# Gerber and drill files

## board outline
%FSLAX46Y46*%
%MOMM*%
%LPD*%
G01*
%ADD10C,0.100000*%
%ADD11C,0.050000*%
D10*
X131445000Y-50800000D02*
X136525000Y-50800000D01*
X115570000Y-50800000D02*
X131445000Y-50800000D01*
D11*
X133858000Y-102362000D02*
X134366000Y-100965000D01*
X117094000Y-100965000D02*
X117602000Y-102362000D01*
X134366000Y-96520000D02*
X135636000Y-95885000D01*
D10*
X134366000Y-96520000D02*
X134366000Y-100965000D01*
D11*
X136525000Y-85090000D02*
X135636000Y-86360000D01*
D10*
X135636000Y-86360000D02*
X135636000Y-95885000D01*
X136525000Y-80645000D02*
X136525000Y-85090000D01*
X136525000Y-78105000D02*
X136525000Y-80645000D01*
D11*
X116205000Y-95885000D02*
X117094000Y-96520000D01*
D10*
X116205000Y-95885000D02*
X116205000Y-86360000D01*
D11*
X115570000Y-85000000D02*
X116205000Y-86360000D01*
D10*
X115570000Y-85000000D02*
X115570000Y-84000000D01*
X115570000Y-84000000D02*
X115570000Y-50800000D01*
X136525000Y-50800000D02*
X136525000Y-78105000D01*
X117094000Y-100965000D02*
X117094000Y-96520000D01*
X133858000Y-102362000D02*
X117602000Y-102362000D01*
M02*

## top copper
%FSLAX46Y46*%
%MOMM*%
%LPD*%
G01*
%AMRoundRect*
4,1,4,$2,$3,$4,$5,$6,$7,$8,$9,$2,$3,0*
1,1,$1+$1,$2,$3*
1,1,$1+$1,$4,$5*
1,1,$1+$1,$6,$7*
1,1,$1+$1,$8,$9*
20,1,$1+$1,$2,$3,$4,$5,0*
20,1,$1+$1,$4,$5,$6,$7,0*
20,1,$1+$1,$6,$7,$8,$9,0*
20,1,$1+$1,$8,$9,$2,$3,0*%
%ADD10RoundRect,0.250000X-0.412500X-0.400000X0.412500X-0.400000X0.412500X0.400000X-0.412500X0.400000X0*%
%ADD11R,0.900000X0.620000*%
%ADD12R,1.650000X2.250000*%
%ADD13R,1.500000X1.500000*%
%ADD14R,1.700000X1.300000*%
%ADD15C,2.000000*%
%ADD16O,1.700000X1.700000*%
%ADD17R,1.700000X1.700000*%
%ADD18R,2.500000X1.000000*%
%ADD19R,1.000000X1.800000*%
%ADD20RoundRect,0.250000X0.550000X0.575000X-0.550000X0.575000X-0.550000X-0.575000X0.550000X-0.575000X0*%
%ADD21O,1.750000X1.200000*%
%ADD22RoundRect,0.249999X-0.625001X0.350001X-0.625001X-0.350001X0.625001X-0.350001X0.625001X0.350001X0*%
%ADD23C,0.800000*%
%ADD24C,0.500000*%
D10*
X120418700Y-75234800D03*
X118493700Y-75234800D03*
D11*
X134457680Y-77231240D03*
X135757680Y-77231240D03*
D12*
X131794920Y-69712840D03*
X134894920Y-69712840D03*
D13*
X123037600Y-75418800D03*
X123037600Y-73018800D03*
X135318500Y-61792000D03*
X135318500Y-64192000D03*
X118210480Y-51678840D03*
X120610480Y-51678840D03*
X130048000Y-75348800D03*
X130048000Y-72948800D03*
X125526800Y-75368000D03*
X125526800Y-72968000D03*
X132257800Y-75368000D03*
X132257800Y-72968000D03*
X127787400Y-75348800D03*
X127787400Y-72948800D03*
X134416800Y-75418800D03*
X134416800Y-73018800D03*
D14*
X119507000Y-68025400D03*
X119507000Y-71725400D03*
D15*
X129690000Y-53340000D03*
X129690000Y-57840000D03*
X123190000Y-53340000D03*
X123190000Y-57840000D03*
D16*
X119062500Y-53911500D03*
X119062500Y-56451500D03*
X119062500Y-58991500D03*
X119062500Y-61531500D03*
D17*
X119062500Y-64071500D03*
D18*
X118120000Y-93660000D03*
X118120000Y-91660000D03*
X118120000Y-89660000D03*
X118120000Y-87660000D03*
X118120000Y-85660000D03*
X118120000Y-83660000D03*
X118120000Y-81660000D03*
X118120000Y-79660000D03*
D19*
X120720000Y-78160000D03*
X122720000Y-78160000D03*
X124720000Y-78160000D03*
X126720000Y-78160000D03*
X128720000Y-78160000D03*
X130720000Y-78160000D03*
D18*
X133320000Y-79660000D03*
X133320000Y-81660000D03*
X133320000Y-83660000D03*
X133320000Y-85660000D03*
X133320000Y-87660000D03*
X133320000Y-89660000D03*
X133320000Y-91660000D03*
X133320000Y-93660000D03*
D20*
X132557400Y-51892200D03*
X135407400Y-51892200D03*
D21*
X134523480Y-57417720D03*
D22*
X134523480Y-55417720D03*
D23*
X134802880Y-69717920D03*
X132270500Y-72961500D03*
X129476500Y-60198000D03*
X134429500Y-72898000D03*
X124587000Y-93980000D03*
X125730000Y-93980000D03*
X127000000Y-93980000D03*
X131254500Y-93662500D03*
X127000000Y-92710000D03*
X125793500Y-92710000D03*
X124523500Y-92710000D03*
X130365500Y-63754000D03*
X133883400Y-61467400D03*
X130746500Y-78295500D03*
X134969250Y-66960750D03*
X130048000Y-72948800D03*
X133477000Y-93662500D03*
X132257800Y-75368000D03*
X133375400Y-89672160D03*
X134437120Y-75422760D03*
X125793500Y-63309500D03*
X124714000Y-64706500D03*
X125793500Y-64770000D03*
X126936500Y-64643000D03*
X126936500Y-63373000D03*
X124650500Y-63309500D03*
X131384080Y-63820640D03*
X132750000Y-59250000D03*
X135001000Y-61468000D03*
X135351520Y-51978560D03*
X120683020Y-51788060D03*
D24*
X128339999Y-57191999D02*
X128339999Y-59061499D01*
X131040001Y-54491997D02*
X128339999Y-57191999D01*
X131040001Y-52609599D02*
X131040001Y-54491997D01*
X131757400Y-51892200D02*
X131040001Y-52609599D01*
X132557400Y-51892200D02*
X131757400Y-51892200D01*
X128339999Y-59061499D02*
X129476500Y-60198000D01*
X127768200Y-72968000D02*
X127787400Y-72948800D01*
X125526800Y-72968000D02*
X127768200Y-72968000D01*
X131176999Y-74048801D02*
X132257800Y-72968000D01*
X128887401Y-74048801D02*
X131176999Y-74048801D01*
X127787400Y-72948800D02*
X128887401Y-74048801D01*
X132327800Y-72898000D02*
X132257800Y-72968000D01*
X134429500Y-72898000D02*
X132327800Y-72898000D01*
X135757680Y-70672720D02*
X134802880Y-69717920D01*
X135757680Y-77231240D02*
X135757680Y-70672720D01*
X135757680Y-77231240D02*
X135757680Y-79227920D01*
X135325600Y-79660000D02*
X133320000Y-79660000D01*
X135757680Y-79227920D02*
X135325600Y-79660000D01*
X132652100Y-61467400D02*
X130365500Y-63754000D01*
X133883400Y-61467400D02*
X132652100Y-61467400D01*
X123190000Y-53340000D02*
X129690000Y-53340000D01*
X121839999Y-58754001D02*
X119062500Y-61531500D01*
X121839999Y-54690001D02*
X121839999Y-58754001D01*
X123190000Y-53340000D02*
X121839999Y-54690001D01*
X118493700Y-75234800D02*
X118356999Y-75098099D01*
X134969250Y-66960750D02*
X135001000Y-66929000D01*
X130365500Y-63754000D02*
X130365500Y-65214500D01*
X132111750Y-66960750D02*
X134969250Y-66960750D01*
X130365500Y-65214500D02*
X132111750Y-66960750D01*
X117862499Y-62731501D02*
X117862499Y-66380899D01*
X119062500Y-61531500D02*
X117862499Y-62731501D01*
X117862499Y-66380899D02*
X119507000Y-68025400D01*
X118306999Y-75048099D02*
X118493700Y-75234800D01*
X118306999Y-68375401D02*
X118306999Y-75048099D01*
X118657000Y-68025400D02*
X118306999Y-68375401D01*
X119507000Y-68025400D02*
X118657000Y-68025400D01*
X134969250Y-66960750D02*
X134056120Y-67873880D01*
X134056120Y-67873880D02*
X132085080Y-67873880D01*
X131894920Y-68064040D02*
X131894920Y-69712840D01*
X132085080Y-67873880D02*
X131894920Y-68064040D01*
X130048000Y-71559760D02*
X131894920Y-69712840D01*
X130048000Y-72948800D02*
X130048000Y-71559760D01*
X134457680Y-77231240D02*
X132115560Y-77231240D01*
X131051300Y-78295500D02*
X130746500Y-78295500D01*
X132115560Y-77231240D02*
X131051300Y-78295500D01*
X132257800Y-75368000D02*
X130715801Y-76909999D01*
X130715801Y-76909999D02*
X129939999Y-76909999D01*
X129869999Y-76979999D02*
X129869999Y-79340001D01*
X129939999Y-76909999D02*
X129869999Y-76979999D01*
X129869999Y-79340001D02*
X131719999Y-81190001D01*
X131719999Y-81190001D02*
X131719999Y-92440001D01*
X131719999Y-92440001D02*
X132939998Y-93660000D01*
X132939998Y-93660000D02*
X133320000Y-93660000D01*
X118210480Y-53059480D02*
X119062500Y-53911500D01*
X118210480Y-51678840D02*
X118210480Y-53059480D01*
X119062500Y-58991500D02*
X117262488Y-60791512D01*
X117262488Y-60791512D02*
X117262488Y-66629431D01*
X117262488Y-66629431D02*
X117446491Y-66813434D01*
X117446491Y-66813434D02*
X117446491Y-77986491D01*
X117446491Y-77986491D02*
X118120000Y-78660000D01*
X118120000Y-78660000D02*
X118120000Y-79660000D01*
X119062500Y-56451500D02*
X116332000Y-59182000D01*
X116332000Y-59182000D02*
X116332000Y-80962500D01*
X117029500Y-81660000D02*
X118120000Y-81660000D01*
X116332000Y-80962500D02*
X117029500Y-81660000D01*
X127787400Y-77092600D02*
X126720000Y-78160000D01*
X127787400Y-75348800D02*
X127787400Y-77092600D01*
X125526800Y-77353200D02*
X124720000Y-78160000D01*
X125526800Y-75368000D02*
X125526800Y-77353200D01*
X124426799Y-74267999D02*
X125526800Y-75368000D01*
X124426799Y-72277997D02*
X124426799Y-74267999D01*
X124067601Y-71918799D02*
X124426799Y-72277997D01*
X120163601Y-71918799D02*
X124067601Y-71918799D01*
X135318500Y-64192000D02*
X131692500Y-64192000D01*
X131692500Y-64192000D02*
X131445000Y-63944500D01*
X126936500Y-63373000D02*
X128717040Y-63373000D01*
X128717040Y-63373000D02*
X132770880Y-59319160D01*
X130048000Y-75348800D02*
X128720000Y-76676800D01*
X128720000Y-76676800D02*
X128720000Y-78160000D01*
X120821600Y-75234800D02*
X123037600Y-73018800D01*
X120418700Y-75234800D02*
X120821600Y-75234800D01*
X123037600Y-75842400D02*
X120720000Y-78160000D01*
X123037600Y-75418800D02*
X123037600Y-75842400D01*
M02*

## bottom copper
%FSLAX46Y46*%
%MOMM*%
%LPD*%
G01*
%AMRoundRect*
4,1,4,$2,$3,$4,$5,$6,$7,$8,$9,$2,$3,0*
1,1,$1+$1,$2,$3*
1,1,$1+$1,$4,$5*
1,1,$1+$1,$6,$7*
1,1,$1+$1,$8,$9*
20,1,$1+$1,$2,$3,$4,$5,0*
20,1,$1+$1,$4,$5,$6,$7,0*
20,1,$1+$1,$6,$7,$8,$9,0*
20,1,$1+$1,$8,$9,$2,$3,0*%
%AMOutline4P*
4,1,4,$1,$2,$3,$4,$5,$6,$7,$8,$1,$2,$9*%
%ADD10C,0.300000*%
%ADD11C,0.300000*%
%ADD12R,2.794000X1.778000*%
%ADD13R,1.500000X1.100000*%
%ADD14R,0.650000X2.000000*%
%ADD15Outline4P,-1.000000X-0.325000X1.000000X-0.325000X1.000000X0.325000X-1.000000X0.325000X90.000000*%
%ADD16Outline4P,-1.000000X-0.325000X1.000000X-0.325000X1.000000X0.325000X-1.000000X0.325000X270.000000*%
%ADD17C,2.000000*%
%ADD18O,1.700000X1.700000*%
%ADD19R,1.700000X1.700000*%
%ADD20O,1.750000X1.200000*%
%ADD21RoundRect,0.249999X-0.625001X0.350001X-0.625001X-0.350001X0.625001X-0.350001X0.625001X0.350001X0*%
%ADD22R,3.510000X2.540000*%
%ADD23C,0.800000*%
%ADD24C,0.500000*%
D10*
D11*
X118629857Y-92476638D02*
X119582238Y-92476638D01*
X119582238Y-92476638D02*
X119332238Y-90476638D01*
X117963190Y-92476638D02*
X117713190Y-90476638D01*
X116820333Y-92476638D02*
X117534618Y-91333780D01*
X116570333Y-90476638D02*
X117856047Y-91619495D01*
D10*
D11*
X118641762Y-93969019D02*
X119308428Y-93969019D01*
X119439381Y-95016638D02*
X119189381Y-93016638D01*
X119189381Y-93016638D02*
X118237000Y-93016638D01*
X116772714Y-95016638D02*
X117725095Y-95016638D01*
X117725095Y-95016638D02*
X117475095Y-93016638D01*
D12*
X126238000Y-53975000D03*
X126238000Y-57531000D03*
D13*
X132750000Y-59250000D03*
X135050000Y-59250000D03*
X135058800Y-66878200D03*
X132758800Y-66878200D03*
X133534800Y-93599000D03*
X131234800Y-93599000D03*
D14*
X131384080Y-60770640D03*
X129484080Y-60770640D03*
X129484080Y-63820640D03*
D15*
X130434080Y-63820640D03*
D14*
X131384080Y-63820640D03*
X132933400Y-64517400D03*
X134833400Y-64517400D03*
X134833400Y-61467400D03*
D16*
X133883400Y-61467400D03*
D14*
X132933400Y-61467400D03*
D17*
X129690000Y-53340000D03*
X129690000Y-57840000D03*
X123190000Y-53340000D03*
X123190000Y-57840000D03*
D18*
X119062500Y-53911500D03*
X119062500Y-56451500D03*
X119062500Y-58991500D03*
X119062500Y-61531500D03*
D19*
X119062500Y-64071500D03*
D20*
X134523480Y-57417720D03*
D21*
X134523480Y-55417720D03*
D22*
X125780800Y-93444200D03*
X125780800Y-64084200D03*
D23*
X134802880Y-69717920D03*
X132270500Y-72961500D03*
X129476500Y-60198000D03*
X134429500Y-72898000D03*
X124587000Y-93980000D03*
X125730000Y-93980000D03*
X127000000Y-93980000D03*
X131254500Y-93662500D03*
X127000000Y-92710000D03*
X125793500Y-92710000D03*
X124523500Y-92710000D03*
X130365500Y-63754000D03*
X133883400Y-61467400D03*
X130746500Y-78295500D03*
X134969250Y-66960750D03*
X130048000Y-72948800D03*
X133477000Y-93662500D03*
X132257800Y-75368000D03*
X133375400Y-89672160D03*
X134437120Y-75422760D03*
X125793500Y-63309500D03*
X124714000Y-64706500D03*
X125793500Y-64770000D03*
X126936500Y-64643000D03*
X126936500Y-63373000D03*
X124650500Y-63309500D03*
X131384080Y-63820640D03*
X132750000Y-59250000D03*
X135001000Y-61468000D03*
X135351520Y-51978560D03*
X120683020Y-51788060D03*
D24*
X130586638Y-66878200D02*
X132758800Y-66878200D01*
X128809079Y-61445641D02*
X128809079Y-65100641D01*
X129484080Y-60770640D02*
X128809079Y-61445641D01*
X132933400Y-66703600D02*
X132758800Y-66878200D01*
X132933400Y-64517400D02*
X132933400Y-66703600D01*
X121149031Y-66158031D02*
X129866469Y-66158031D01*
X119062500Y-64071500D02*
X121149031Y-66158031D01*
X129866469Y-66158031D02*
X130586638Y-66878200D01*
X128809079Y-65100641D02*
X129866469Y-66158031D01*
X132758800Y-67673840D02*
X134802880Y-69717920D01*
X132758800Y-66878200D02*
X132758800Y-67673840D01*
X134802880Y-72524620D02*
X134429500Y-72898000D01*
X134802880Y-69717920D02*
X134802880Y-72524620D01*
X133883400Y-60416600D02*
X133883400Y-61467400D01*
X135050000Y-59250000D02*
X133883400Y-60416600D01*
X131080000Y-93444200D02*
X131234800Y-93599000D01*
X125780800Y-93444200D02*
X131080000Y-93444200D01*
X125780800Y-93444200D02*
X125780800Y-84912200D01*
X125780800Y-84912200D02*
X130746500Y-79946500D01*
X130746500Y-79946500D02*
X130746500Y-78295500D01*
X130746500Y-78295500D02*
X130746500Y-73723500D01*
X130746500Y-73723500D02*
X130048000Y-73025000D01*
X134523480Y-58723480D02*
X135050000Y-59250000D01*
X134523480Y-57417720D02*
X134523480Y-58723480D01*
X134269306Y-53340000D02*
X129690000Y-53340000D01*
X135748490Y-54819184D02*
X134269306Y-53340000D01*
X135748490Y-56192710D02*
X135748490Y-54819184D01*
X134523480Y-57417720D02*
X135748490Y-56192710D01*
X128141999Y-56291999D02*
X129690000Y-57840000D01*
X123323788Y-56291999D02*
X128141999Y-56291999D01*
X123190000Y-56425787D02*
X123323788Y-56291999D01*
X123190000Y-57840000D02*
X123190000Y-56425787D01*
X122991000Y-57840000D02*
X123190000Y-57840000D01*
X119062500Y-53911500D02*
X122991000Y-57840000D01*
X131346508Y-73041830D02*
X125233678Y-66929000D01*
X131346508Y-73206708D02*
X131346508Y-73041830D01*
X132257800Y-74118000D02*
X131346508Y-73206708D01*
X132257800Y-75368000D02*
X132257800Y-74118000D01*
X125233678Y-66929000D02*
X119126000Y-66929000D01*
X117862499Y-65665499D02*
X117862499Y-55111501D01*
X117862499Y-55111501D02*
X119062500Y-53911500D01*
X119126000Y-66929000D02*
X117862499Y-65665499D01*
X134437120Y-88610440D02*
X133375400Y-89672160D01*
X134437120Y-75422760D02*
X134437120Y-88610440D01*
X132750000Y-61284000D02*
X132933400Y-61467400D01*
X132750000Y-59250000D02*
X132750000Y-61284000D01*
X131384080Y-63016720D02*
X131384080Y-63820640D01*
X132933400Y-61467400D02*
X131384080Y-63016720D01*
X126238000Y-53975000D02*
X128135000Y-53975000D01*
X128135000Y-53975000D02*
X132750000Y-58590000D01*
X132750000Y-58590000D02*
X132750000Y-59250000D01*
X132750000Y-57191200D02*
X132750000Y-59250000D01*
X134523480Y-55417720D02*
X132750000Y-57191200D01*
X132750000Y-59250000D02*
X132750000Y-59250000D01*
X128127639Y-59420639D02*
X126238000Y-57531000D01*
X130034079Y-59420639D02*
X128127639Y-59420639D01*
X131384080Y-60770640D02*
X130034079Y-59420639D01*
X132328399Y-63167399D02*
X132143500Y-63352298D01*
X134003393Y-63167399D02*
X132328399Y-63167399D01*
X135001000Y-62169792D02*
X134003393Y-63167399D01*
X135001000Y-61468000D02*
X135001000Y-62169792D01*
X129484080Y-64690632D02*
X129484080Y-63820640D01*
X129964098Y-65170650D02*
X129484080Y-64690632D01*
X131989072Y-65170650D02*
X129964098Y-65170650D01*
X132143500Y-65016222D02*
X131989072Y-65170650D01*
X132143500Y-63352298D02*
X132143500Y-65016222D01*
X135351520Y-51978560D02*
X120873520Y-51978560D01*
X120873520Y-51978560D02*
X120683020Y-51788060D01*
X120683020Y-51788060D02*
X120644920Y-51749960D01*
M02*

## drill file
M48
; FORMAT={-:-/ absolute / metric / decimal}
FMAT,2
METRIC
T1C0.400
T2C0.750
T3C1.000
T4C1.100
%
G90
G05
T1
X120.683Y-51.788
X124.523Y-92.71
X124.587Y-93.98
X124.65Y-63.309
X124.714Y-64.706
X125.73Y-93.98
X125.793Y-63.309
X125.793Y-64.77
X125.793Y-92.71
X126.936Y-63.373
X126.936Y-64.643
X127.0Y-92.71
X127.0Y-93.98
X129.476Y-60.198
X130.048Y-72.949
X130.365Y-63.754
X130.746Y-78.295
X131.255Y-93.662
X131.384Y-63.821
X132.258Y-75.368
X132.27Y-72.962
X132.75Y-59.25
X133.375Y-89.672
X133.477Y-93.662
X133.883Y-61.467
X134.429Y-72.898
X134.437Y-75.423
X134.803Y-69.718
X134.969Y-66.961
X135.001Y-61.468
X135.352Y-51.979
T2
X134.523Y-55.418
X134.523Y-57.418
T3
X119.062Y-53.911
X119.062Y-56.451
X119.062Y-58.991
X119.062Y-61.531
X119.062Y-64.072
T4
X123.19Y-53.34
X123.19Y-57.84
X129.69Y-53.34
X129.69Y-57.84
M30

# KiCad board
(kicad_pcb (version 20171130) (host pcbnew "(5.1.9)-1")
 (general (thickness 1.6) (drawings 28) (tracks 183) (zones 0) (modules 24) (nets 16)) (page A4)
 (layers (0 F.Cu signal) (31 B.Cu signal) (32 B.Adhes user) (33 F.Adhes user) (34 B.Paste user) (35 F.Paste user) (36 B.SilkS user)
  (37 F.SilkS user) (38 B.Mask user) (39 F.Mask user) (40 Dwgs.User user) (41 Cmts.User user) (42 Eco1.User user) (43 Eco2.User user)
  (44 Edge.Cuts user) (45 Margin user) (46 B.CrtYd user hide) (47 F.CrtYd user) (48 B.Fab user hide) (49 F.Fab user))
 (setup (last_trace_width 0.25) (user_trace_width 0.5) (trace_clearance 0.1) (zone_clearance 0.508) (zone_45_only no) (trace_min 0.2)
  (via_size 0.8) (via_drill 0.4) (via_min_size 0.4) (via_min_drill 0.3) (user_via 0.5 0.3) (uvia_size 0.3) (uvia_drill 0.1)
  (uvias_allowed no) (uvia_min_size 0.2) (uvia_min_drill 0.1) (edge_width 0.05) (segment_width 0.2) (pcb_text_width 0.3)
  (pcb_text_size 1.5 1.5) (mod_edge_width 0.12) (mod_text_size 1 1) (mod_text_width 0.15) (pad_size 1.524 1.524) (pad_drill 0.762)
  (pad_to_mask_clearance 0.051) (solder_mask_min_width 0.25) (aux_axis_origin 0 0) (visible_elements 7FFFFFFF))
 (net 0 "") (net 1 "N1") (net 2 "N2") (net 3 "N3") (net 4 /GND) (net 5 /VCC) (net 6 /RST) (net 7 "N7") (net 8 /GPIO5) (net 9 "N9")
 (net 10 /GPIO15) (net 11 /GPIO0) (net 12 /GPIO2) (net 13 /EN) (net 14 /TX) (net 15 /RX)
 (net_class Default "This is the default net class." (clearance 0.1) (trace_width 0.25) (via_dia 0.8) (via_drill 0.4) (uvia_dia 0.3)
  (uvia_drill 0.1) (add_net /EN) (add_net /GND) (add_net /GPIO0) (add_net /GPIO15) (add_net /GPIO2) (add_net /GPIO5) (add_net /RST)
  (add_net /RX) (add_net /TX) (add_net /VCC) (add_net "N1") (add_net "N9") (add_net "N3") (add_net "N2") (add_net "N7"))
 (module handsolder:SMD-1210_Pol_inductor (layer B.Cu) (at 126.238 55.753 270)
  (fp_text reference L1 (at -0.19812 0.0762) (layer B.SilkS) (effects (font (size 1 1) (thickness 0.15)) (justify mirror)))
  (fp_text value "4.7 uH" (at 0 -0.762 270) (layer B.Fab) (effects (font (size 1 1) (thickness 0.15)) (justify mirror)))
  (pad 1 smd rect (at -1.778 0 270) (size 1.778 2.794) (layers B.Cu B.Paste B.Mask) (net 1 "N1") (zone_connect 2))
  (pad 2 smd rect (at 1.778 0 270) (size 1.778 2.794) (layers B.Cu B.Paste B.Mask) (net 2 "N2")))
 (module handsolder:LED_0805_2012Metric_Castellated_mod (layer F.Cu) (at 119.4562 75.2348)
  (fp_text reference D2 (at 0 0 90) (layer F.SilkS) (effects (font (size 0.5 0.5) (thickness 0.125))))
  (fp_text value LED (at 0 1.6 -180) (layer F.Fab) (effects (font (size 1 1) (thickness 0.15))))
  (pad 2 smd roundrect (at 0.9625 0) (size 1.325 1.3) (layers F.Cu F.Paste F.Mask) (roundrect_rratio 0.1923076923076923) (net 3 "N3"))
  (pad 1 smd roundrect (at -0.9625 0) (size 1.325 1.3) (layers F.Cu F.Paste F.Mask) (roundrect_rratio 0.1923076923076923) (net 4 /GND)))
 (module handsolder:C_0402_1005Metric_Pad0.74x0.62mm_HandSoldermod (layer F.Cu) (at 135.10768 77.23124 180)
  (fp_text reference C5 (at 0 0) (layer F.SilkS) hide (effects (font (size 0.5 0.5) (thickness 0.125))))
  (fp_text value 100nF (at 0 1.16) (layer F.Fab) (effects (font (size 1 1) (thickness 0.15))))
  (pad 2 smd rect (at 0.65 0 180) (size 0.9 0.62) (layers F.Cu F.Paste F.Mask) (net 4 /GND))
  (pad 1 smd rect (at -0.65 0 180) (size 0.9 0.62) (layers F.Cu F.Paste F.Mask) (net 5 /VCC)))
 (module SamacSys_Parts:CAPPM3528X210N (layer F.Cu) (at 133.34492 69.71284 180)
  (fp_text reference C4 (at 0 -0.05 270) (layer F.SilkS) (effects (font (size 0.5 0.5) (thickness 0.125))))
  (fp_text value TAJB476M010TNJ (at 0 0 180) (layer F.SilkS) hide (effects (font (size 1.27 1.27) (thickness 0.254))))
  (pad 2 smd rect (at 1.55 0 180) (size 1.65 2.25) (layers F.Cu F.Paste F.Mask) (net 4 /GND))
  (pad 1 smd rect (at -1.55 0 180) (size 1.65 2.25) (layers F.Cu F.Paste F.Mask) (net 5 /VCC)))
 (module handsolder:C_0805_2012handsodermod (layer B.Cu) (at 133.9 59.25 180)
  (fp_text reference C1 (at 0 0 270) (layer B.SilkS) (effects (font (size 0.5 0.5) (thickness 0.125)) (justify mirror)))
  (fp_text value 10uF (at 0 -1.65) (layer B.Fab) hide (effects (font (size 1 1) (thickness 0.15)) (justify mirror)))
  (pad 2 smd rect (at 1.15 0 180) (size 1.5 1.1) (layers B.Cu B.Paste B.Mask) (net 1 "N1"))
  (pad 1 smd rect (at -1.15 0 180) (size 1.5 1.1) (layers B.Cu B.Paste B.Mask) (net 4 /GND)))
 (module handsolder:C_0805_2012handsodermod (layer B.Cu) (at 133.9088 66.8782)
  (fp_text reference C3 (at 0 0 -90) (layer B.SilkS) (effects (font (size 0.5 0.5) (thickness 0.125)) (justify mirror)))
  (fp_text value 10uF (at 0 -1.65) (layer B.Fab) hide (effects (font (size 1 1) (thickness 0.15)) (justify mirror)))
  (pad 2 smd rect (at 1.15 0) (size 1.5 1.1) (layers B.Cu B.Paste B.Mask) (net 4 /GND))
  (pad 1 smd rect (at -1.15 0) (size 1.5 1.1) (layers B.Cu B.Paste B.Mask) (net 5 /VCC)))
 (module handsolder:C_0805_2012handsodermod (layer B.Cu) (at 132.3848 93.599)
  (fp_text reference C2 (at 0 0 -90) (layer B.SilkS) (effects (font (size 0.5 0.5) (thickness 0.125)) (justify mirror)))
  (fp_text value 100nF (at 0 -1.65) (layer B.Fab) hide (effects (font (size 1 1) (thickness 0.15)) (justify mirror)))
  (pad 2 smd rect (at 1.15 0) (size 1.5 1.1) (layers B.Cu B.Paste B.Mask) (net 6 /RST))
  (pad 1 smd rect (at -1.15 0) (size 1.5 1.1) (layers B.Cu B.Paste B.Mask) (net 4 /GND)))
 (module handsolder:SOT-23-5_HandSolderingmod (layer B.Cu) (at 130.43408 62.27064 90)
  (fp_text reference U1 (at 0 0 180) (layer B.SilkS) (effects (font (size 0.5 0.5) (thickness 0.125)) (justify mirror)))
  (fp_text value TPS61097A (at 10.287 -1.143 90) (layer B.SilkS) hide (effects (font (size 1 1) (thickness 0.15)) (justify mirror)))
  (pad 5 smd rect (at 1.5 0.95 90) (size 2 0.65) (layers B.Cu B.Paste B.Mask) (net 2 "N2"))
  (pad 4 smd rect (at 1.5 -0.95 90) (size 2 0.65) (layers B.Cu B.Paste B.Mask) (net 5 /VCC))
  (pad 3 smd rect (at -1.55 -0.95 90) (size 2 0.65) (layers B.Cu B.Paste B.Mask) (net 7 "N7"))
  (pad 2 smd trapezoid (at -1.55 0 90) (size 2 0.65) (layers B.Cu B.Paste B.Mask) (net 4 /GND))
  (pad 1 smd rect (at -1.55 0.95 90) (size 2 0.65) (layers B.Cu B.Paste B.Mask) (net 1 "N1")))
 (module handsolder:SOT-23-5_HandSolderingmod (layer B.Cu) (at 133.8834 63.0174 270)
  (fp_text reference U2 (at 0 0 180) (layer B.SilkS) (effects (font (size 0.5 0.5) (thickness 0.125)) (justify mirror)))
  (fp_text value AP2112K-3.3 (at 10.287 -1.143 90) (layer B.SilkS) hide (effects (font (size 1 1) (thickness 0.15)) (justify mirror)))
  (pad 5 smd rect (at 1.5 0.95 270) (size 2 0.65) (layers B.Cu B.Paste B.Mask) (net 5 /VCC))
  (pad 4 smd rect (at 1.5 -0.95 270) (size 2 0.65) (layers B.Cu B.Paste B.Mask))
  (pad 3 smd rect (at -1.55 -0.95 270) (size 2 0.65) (layers B.Cu B.Paste B.Mask) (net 7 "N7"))
  (pad 2 smd trapezoid (at -1.55 0 270) (size 2 0.65) (layers B.Cu B.Paste B.Mask) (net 4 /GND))
  (pad 1 smd rect (at -1.55 0.95 270) (size 2 0.65) (layers B.Cu B.Paste B.Mask) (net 1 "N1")))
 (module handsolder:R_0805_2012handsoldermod (layer F.Cu) (at 123.0376 74.2188 270)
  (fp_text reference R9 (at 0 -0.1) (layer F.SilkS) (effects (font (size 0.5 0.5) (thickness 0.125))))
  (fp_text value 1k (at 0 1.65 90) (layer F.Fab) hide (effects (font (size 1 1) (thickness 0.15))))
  (pad 2 smd rect (at 1.2 0 270) (size 1.5 1.5) (layers F.Cu F.Paste F.Mask) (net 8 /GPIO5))
  (pad 1 smd rect (at -1.2 0 270) (size 1.5 1.5) (layers F.Cu F.Paste F.Mask) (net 3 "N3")))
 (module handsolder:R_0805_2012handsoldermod (layer F.Cu) (at 135.3185 62.992 90)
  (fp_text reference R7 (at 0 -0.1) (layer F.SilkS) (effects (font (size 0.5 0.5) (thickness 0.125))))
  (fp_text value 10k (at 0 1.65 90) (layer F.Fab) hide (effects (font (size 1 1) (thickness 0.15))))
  (pad 2 smd rect (at 1.2 0 90) (size 1.5 1.5) (layers F.Cu F.Paste F.Mask) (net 7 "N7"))
  (pad 1 smd rect (at -1.2 0 90) (size 1.5 1.5) (layers F.Cu F.Paste F.Mask) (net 1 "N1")))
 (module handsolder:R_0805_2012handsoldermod (layer F.Cu) (at 119.41048 51.67884 180)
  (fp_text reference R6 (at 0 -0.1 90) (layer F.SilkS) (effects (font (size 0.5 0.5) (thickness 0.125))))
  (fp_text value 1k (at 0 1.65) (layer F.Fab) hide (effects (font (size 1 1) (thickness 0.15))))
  (pad 2 smd rect (at 1.2 0 180) (size 1.5 1.5) (layers F.Cu F.Paste F.Mask) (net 6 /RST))
  (pad 1 smd rect (at -1.2 0 180) (size 1.5 1.5) (layers F.Cu F.Paste F.Mask) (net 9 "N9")))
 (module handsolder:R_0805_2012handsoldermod (layer F.Cu) (at 130.048 74.1488 270)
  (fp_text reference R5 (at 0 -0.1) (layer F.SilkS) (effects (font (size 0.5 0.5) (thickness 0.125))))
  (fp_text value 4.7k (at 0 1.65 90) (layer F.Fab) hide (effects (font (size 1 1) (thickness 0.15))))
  (pad 2 smd rect (at 1.2 0 270) (size 1.5 1.5) (layers F.Cu F.Paste F.Mask) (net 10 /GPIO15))
  (pad 1 smd rect (at -1.2 0 270) (size 1.5 1.5) (layers F.Cu F.Paste F.Mask) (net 4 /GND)))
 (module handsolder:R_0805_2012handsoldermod (layer F.Cu) (at 125.5268 74.168 270)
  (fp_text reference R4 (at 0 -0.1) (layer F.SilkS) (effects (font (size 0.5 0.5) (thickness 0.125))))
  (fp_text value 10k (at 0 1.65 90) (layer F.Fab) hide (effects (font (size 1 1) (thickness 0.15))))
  (pad 2 smd rect (at 1.2 0 270) (size 1.5 1.5) (layers F.Cu F.Paste F.Mask) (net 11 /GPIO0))
  (pad 1 smd rect (at -1.2 0 270) (size 1.5 1.5) (layers F.Cu F.Paste F.Mask) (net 5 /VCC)))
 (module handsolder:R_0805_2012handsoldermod (layer F.Cu) (at 132.2578 74.168 270)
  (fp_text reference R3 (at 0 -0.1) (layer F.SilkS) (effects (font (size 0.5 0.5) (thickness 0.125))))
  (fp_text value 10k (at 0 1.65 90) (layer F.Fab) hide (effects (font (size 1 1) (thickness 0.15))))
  (pad 2 smd rect (at 1.2 0 270) (size 1.5 1.5) (layers F.Cu F.Paste F.Mask) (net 6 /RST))
  (pad 1 smd rect (at -1.2 0 270) (size 1.5 1.5) (layers F.Cu F.Paste F.Mask) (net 5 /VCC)))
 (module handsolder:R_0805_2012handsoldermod (layer F.Cu) (at 127.7874 74.1488 270)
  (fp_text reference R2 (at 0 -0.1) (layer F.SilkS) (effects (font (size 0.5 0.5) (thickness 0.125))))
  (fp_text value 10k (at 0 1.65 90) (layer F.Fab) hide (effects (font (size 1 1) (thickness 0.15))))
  (pad 2 smd rect (at 1.2 0 270) (size 1.5 1.5) (layers F.Cu F.Paste F.Mask) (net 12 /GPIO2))
  (pad 1 smd rect (at -1.2 0 270) (size 1.5 1.5) (layers F.Cu F.Paste F.Mask) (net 5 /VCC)))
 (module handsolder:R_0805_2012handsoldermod (layer F.Cu) (at 134.4168 74.2188 270)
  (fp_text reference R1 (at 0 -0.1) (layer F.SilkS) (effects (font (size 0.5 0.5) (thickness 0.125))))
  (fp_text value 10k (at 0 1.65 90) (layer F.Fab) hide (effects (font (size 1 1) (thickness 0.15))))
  (pad 2 smd rect (at 1.2 0 270) (size 1.5 1.5) (layers F.Cu F.Paste F.Mask) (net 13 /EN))
  (pad 1 smd rect (at -1.2 0 270) (size 1.5 1.5) (layers F.Cu F.Paste F.Mask) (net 5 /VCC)))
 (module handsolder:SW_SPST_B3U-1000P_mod (layer F.Cu) (at 119.507 69.8754 90)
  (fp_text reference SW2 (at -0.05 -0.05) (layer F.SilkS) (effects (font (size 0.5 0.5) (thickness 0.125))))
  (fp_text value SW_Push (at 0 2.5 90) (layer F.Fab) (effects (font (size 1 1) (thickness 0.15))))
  (pad 2 smd rect (at 1.85 0 90) (size 1.3 1.7) (layers F.Cu F.Paste F.Mask) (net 4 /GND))
  (pad 1 smd rect (at -1.85 0 90) (size 1.3 1.7) (layers F.Cu F.Paste F.Mask) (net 11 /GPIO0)))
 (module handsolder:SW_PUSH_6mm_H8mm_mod (layer F.Cu) (at 123.19 53.34)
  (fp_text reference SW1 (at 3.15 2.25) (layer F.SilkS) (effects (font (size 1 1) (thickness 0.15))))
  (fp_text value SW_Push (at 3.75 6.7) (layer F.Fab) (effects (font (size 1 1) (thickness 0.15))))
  (pad 1 thru_hole circle (at 6.5 0 90) (size 2 2) (drill 1.1) (layers *.Cu *.Mask) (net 4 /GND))
  (pad 2 thru_hole circle (at 6.5 4.5 90) (size 2 2) (drill 1.1) (layers *.Cu *.Mask) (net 6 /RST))
  (pad 1 thru_hole circle (at 0 0 90) (size 2 2) (drill 1.1) (layers *.Cu *.Mask) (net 4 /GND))
  (pad 2 thru_hole circle (at 0 4.5 90) (size 2 2) (drill 1.1) (layers *.Cu *.Mask) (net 6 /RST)))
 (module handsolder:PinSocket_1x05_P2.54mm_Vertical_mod (layer F.Cu) (at 119.0625 64.0715 180)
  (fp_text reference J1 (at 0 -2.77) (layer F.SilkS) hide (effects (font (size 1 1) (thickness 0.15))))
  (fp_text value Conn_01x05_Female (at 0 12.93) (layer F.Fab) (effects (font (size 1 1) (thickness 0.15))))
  (pad 5 thru_hole oval (at 0 10.16 180) (size 1.7 1.7) (drill 1) (layers *.Cu *.Mask) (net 6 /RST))
  (pad 4 thru_hole oval (at 0 7.62 180) (size 1.7 1.7) (drill 1) (layers *.Cu *.Mask) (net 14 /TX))
  (pad 3 thru_hole oval (at 0 5.08 180) (size 1.7 1.7) (drill 1) (layers *.Cu *.Mask) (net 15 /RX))
  (pad 2 thru_hole oval (at 0 2.54 180) (size 1.7 1.7) (drill 1) (layers *.Cu *.Mask) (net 4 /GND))
  (pad 1 thru_hole rect (at 0 0 180) (size 1.7 1.7) (drill 1) (layers *.Cu *.Mask) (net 5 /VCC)))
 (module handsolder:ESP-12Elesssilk (layer F.Cu) (at 125.72 90.16 180)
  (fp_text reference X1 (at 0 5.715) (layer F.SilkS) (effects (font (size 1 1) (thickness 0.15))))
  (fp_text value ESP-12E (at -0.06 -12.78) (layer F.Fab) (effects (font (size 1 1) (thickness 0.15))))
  (pad 22 smd rect (at 7.6 -3.5 180) (size 2.5 1) (layers F.Cu F.Paste F.Mask))
  (pad 21 smd rect (at 7.6 -1.5 180) (size 2.5 1) (layers F.Cu F.Paste F.Mask))
  (pad 20 smd rect (at 7.6 0.5 180) (size 2.5 1) (layers F.Cu F.Paste F.Mask))
  (pad 19 smd rect (at 7.6 2.5 180) (size 2.5 1) (layers F.Cu F.Paste F.Mask))
  (pad 18 smd rect (at 7.6 4.5 180) (size 2.5 1) (layers F.Cu F.Paste F.Mask))
  (pad 17 smd rect (at 7.6 6.5 180) (size 2.5 1) (layers F.Cu F.Paste F.Mask))
  (pad 16 smd rect (at 7.6 8.5 180) (size 2.5 1) (layers F.Cu F.Paste F.Mask) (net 14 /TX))
  (pad 15 smd rect (at 7.6 10.5 180) (size 2.5 1) (layers F.Cu F.Paste F.Mask) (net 15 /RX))
  (pad 14 smd rect (at 5 12 180) (size 1 1.8) (layers F.Cu F.Paste F.Mask) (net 8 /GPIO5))
  (pad 13 smd rect (at 3 12 180) (size 1 1.8) (layers F.Cu F.Paste F.Mask))
  (pad 12 smd rect (at 1 12 180) (size 1 1.8) (layers F.Cu F.Paste F.Mask) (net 11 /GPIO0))
  (pad 11 smd rect (at -1 12 180) (size 1 1.8) (layers F.Cu F.Paste F.Mask) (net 12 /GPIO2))
  (pad 10 smd rect (at -3 12 180) (size 1 1.8) (layers F.Cu F.Paste F.Mask) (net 10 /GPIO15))
  (pad 9 smd rect (at -5 12 180) (size 1 1.8) (layers F.Cu F.Paste F.Mask) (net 4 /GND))
  (pad 8 smd rect (at -7.6 10.5 180) (size 2.5 1) (layers F.Cu F.Paste F.Mask) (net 5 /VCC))
  (pad 7 smd rect (at -7.6 8.5 180) (size 2.5 1) (layers F.Cu F.Paste F.Mask))
  (pad 6 smd rect (at -7.6 6.5 180) (size 2.5 1) (layers F.Cu F.Paste F.Mask))
  (pad 5 smd rect (at -7.6 4.5 180) (size 2.5 1) (layers F.Cu F.Paste F.Mask))
  (pad 4 smd rect (at -7.6 2.5 180) (size 2.5 1) (layers F.Cu F.Paste F.Mask))
  (pad 3 smd rect (at -7.6 0.5 180) (size 2.5 1) (layers F.Cu F.Paste F.Mask) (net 13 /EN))
  (pad 2 smd rect (at -7.6 -1.5 180) (size 2.5 1) (layers F.Cu F.Paste F.Mask))
  (pad 1 smd rect (at -7.6 -3.5 180) (size 2.5 1) (layers F.Cu F.Paste F.Mask) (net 6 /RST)))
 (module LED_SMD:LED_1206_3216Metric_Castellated (layer F.Cu) (at 133.9824 51.8922 180)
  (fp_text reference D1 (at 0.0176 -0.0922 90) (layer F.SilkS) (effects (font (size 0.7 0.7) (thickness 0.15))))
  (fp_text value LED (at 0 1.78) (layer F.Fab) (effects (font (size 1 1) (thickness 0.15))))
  (pad 2 smd roundrect (at 1.425 0 180) (size 1.6 1.65) (layers F.Cu F.Paste F.Mask) (roundrect_rratio 0.15625) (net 5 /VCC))
  (pad 1 smd roundrect (at -1.425 0 180) (size 1.6 1.65) (layers F.Cu F.Paste F.Mask) (roundrect_rratio 0.15625) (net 9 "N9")))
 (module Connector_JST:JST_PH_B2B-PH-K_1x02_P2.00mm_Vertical (layer F.Cu) (at 134.52348 55.41772 270)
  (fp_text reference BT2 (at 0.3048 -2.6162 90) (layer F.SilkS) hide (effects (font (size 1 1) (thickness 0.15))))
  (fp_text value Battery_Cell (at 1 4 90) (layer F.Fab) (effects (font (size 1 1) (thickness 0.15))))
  (pad 2 thru_hole oval (at 2 0 270) (size 1.2 1.75) (drill 0.75) (layers *.Cu *.Mask) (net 4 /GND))
  (pad 1 thru_hole roundrect (at 0 0 270) (size 1.2 1.75) (drill 0.75) (layers *.Cu *.Mask) (roundrect_rratio 0.2083325) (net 1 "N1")))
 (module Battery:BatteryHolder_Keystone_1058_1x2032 (layer B.Cu) (at 125.7808 78.7642 270)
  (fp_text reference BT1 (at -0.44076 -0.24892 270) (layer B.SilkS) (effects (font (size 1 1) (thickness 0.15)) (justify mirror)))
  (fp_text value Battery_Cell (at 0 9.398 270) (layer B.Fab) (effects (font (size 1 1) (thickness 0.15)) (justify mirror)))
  (pad 2 smd rect (at 14.68 0 270) (size 2.54 3.51) (layers B.Cu B.Paste B.Mask) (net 4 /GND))
  (pad 1 smd rect (at -14.68 0 270) (size 2.54 3.51) (layers B.Cu B.Paste B.Mask) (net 1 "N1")))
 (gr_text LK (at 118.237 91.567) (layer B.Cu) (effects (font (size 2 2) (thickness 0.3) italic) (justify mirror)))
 (gr_line (start 131.445 50.8) (end 136.525 50.8) (layer Edge.Cuts) (width 0.1))
 (gr_line (start 115.57 50.8) (end 131.445 50.8) (layer Edge.Cuts) (width 0.1))
 (gr_line (start 133.858 102.362) (end 134.366 100.965) (layer Edge.Cuts) (width 0.05))
 (gr_line (start 117.094 100.965) (end 117.602 102.362) (layer Edge.Cuts) (width 0.05))
 (gr_line (start 134.366 96.52) (end 135.636 95.885) (layer Edge.Cuts) (width 0.05))
 (gr_line (start 134.366 96.52) (end 134.366 100.965) (layer Edge.Cuts) (width 0.1))
 (gr_line (start 136.525 85.09) (end 135.636 86.36) (layer Edge.Cuts) (width 0.05))
 (gr_line (start 135.636 86.36) (end 135.636 95.885) (layer Edge.Cuts) (width 0.1))
 (gr_line (start 136.525 80.645) (end 136.525 85.09) (layer Edge.Cuts) (width 0.1))
 (gr_line (start 136.525 78.105) (end 136.525 80.645) (layer Edge.Cuts) (width 0.1))
 (gr_line (start 116.205 95.885) (end 117.094 96.52) (layer Edge.Cuts) (width 0.05))
 (gr_line (start 116.205 95.885) (end 116.205 86.36) (layer Edge.Cuts) (width 0.1))
 (gr_line (start 115.57 85) (end 116.205 86.36) (layer Edge.Cuts) (width 0.05))
 (gr_line (start 115.57 85) (end 115.57 84) (layer Edge.Cuts) (width 0.1))
 (gr_line (start 115.57 84) (end 115.57 50.8) (layer Edge.Cuts) (width 0.1))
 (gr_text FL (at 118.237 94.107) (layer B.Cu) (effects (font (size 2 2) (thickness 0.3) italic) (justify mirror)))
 (gr_line (start 136.525 50.8) (end 136.525 78.105) (layer Edge.Cuts) (width 0.1))
 (gr_line (start 117.094 100.965) (end 117.094 96.52) (layer Edge.Cuts) (width 0.1))
 (gr_line (start 133.858 102.362) (end 117.602 102.362) (layer Edge.Cuts) (width 0.1))
 (via (at 134.80288 69.71792) (size 0.8) (drill 0.4) (layers F.Cu B.Cu) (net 5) (status 30))
 (via (at 132.2705 72.9615) (size 0.8) (drill 0.4) (layers F.Cu B.Cu) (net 5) (status 30))
 (segment (start 130.586638 66.8782) (end 132.7588 66.8782) (width 0.5) (layer B.Cu) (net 5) (status 20))
 (segment (start 128.809079 61.445641) (end 128.809079 65.100641) (width 0.5) (layer B.Cu) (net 5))
 (segment (start 129.48408 60.77064) (end 128.809079 61.445641) (width 0.5) (layer B.Cu) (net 5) (status 10))
 (segment (start 132.9334 66.7036) (end 132.7588 66.8782) (width 0.5) (layer B.Cu) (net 5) (status 30))
 (segment (start 132.9334 64.5174) (end 132.9334 66.7036) (width 0.5) (layer B.Cu) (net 5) (status 30))
 (segment (start 128.339999 57.191999) (end 128.339999 59.061499) (width 0.5) (layer F.Cu) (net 5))
 (segment (start 131.040001 54.491997) (end 128.339999 57.191999) (width 0.5) (layer F.Cu) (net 5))
 (segment (start 131.040001 52.609599) (end 131.040001 54.491997) (width 0.5) (layer F.Cu) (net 5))
 (segment (start 131.7574 51.8922) (end 131.040001 52.609599) (width 0.5) (layer F.Cu) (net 5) (status 10))
 (segment (start 132.5574 51.8922) (end 131.7574 51.8922) (width 0.5) (layer F.Cu) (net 5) (status 30))
 (segment (start 128.339999 59.061499) (end 129.4765 60.198) (width 0.5) (layer F.Cu) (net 5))
 (via (at 129.4765 60.198) (size 0.8) (drill 0.4) (layers F.Cu B.Cu) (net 5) (status 30))
 (via (at 134.4295 72.898) (size 0.8) (drill 0.4) (layers F.Cu B.Cu) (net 5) (status 30))
 (segment (start 127.7682 72.968) (end 127.7874 72.9488) (width 0.5) (layer F.Cu) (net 5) (status 30))
 (segment (start 125.5268 72.968) (end 127.7682 72.968) (width 0.5) (layer F.Cu) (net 5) (status 30))
 (segment (start 131.176999 74.048801) (end 132.2578 72.968) (width 0.5) (layer F.Cu) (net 5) (status 20))
 (segment (start 128.887401 74.048801) (end 131.176999 74.048801) (width 0.5) (layer F.Cu) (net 5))
 (segment (start 127.7874 72.9488) (end 128.887401 74.048801) (width 0.5) (layer F.Cu) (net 5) (status 10))
 (segment (start 121.149031 66.158031) (end 129.866469 66.158031) (width 0.5) (layer B.Cu) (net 5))
 (segment (start 119.0625 64.0715) (end 121.149031 66.158031) (width 0.5) (layer B.Cu) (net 5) (status 10))
 (segment (start 129.866469 66.158031) (end 130.586638 66.8782) (width 0.5) (layer B.Cu) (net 5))
 (segment (start 128.809079 65.100641) (end 129.866469 66.158031) (width 0.5) (layer B.Cu) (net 5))
 (segment (start 132.7588 67.67384) (end 134.80288 69.71792) (width 0.5) (layer B.Cu) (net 5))
 (segment (start 132.7588 66.8782) (end 132.7588 67.67384) (width 0.5) (layer B.Cu) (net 5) (status 10))
 (segment (start 134.80288 72.52462) (end 134.4295 72.898) (width 0.5) (layer B.Cu) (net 5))
 (segment (start 134.80288 69.71792) (end 134.80288 72.52462) (width 0.5) (layer B.Cu) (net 5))
 (segment (start 132.3278 72.898) (end 132.2578 72.968) (width 0.5) (layer F.Cu) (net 5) (status 30))
 (segment (start 134.4295 72.898) (end 132.3278 72.898) (width 0.5) (layer F.Cu) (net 5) (status 30))
 (segment (start 135.75768 70.67272) (end 134.80288 69.71792) (width 0.5) (layer F.Cu) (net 5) (status 20))
 (segment (start 135.75768 77.23124) (end 135.75768 70.67272) (width 0.5) (layer F.Cu) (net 5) (status 10))
 (segment (start 135.75768 77.23124) (end 135.75768 79.22792) (width 0.5) (layer F.Cu) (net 5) (status 10))
 (segment (start 135.3256 79.66) (end 133.32 79.66) (width 0.5) (layer F.Cu) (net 5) (status 20))
 (segment (start 135.75768 79.22792) (end 135.3256 79.66) (width 0.5) (layer F.Cu) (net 5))
 (via (at 124.587 93.98) (size 0.8) (drill 0.4) (layers F.Cu B.Cu) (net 4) (status 30))
 (via (at 125.73 93.98) (size 0.8) (drill 0.4) (layers F.Cu B.Cu) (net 4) (status 30))
 (via (at 127 93.98) (size 0.8) (drill 0.4) (layers F.Cu B.Cu) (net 4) (status 30))
 (via (at 131.2545 93.6625) (size 0.8) (drill 0.4) (layers F.Cu B.Cu) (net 4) (status 30))
 (via (at 127 92.71) (size 0.8) (drill 0.4) (layers F.Cu B.Cu) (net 4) (status 30))
 (via (at 125.7935 92.71) (size 0.8) (drill 0.4) (layers F.Cu B.Cu) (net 4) (status 30))
 (via (at 124.5235 92.71) (size 0.8) (drill 0.4) (layers F.Cu B.Cu) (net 4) (status 30))
 (via (at 130.3655 63.754) (size 0.8) (drill 0.4) (layers F.Cu B.Cu) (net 4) (status 30))
 (segment (start 133.8834 60.4166) (end 133.8834 61.4674) (width 0.5) (layer B.Cu) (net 4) (status 20))
 (segment (start 135.05 59.25) (end 133.8834 60.4166) (width 0.5) (layer B.Cu) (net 4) (status 10))
 (via (at 133.8834 61.4674) (size 0.8) (drill 0.4) (layers F.Cu B.Cu) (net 4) (status 30))
 (segment (start 132.6521 61.4674) (end 130.3655 63.754) (width 0.5) (layer F.Cu) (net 4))
 (segment (start 133.8834 61.4674) (end 132.6521 61.4674) (width 0.5) (layer F.Cu) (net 4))
 (segment (start 123.19 53.34) (end 129.69 53.34) (width 0.5) (layer F.Cu) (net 4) (status 30))
 (segment (start 121.839999 58.754001) (end 119.0625 61.5315) (width 0.5) (layer F.Cu) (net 4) (status 20))
 (segment (start 121.839999 54.690001) (end 121.839999 58.754001) (width 0.5) (layer F.Cu) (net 4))
 (segment (start 123.19 53.34) (end 121.839999 54.690001) (width 0.5) (layer F.Cu) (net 4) (status 10))
 (segment (start 131.08 93.4442) (end 131.2348 93.599) (width 0.5) (layer B.Cu) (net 4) (status 30))
 (segment (start 125.7808 93.4442) (end 131.08 93.4442) (width 0.5) (layer B.Cu) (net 4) (status 30))
 (segment (start 125.7808 93.4442) (end 125.7808 84.9122) (width 0.5) (layer B.Cu) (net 4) (status 10))
 (segment (start 125.7808 84.9122) (end 130.7465 79.9465) (width 0.5) (layer B.Cu) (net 4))
 (segment (start 130.7465 79.9465) (end 130.7465 78.2955) (width 0.5) (layer B.Cu) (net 4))
 (via (at 130.7465 78.2955) (size 0.8) (drill 0.4) (layers F.Cu B.Cu) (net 4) (status 30))
 (segment (start 118.4937 75.2348) (end 118.356999 75.098099) (width 0.5) (layer F.Cu) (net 4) (status 30))
 (segment (start 134.96925 66.96075) (end 135.001 66.929) (width 0.5) (layer F.Cu) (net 4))
 (via (at 134.96925 66.96075) (size 0.8) (drill 0.4) (layers F.Cu B.Cu) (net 4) (status 30))
 (segment (start 130.7465 78.2955) (end 130.7465 73.7235) (width 0.5) (layer B.Cu) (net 4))
 (segment (start 130.7465 73.7235) (end 130.048 73.025) (width 0.5) (layer B.Cu) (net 4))
 (via (at 130.048 72.9488) (size 0.8) (drill 0.4) (layers F.Cu B.Cu) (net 4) (status 30))
 (segment (start 130.3655 63.754) (end 130.3655 65.2145) (width 0.5) (layer F.Cu) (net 4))
 (segment (start 132.11175 66.96075) (end 134.96925 66.96075) (width 0.5) (layer F.Cu) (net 4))
 (segment (start 130.3655 65.2145) (end 132.11175 66.96075) (width 0.5) (layer F.Cu) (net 4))
 (segment (start 117.862499 62.731501) (end 117.862499 66.380899) (width 0.5) (layer F.Cu) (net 4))
 (segment (start 119.0625 61.5315) (end 117.862499 62.731501) (width 0.5) (layer F.Cu) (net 4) (status 10))
 (segment (start 117.862499 66.380899) (end 119.507 68.0254) (width 0.5) (layer F.Cu) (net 4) (status 20))
 (segment (start 118.306999 75.048099) (end 118.4937 75.2348) (width 0.5) (layer F.Cu) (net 4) (status 30))
 (segment (start 118.306999 68.375401) (end 118.306999 75.048099) (width 0.5) (layer F.Cu) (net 4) (status 20))
 (segment (start 118.657 68.0254) (end 118.306999 68.375401) (width 0.5) (layer F.Cu) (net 4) (status 10))
 (segment (start 119.507 68.0254) (end 118.657 68.0254) (width 0.5) (layer F.Cu) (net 4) (status 30))
 (segment (start 134.96925 66.96075) (end 134.05612 67.87388) (width 0.5) (layer F.Cu) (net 4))
 (segment (start 134.05612 67.87388) (end 132.08508 67.87388) (width 0.5) (layer F.Cu) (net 4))
 (segment (start 131.89492 68.06404) (end 131.89492 69.71284) (width 0.5) (layer F.Cu) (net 4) (status 20))
 (segment (start 132.08508 67.87388) (end 131.89492 68.06404) (width 0.5) (layer F.Cu) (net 4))
 (segment (start 130.048 71.55976) (end 131.89492 69.71284) (width 0.5) (layer F.Cu) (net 4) (status 20))
 (segment (start 130.048 72.9488) (end 130.048 71.55976) (width 0.5) (layer F.Cu) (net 4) (status 10))
 (segment (start 134.45768 77.23124) (end 132.11556 77.23124) (width 0.5) (layer F.Cu) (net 4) (status 10))
 (segment (start 131.0513 78.2955) (end 130.7465 78.2955) (width 0.5) (layer F.Cu) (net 4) (status 30))
 (segment (start 132.11556 77.23124) (end 131.0513 78.2955) (width 0.5) (layer F.Cu) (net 4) (status 20))
 (segment (start 134.52348 58.72348) (end 135.05 59.25) (width 0.5) (layer B.Cu) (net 4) (status 30))
 (segment (start 134.52348 57.41772) (end 134.52348 58.72348) (width 0.5) (layer B.Cu) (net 4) (status 30))
 (segment (start 134.269306 53.34) (end 129.69 53.34) (width 0.5) (layer B.Cu) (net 4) (status 20))
 (segment (start 135.74849 54.819184) (end 134.269306 53.34) (width 0.5) (layer B.Cu) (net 4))
 (segment (start 135.74849 56.19271) (end 135.74849 54.819184) (width 0.5) (layer B.Cu) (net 4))
 (segment (start 134.52348 57.41772) (end 135.74849 56.19271) (width 0.5) (layer B.Cu) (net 4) (status 10))
 (via (at 133.477 93.6625) (size 0.8) (drill 0.4) (layers F.Cu B.Cu) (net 6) (status 30))
 (segment (start 128.141999 56.291999) (end 129.69 57.84) (width 0.5) (layer B.Cu) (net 6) (status 20))
 (segment (start 123.323788 56.291999) (end 128.141999 56.291999) (width 0.5) (layer B.Cu) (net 6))
 (segment (start 123.19 56.425787) (end 123.323788 56.291999) (width 0.5) (layer B.Cu) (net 6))
 (segment (start 123.19 57.84) (end 123.19 56.425787) (width 0.5) (layer B.Cu) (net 6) (status 10))
 (segment (start 122.991 57.84) (end 123.19 57.84) (width 0.5) (layer B.Cu) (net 6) (status 30))
 (segment (start 119.0625 53.9115) (end 122.991 57.84) (width 0.5) (layer B.Cu) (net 6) (status 30))
 (via (at 132.2578 75.368) (size 0.8) (drill 0.4) (layers F.Cu B.Cu) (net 6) (status 30))
 (segment (start 131.346508 73.04183) (end 125.233678 66.929) (width 0.5) (layer B.Cu) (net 6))
 (segment (start 131.346508 73.206708) (end 131.346508 73.04183) (width 0.5) (layer B.Cu) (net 6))
 (segment (start 132.2578 74.118) (end 131.346508 73.206708) (width 0.5) (layer B.Cu) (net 6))
 (segment (start 132.2578 75.368) (end 132.2578 74.118) (width 0.5) (layer B.Cu) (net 6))
 (segment (start 125.233678 66.929) (end 119.126 66.929) (width 0.5) (layer B.Cu) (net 6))
 (segment (start 117.862499 65.665499) (end 117.862499 55.111501) (width 0.5) (layer B.Cu) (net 6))
 (segment (start 117.862499 55.111501) (end 119.0625 53.9115) (width 0.5) (layer B.Cu) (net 6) (status 20))
 (segment (start 119.126 66.929) (end 117.862499 65.665499) (width 0.5) (layer B.Cu) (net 6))
 (segment (start 132.2578 75.368) (end 130.715801 76.909999) (width 0.5) (layer F.Cu) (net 6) (status 10))
 (segment (start 130.715801 76.909999) (end 129.939999 76.909999) (width 0.5) (layer F.Cu) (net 6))
 (segment (start 129.869999 76.979999) (end 129.869999 79.340001) (width 0.5) (layer F.Cu) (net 6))
 (segment (start 129.939999 76.909999) (end 129.869999 76.979999) (width 0.5) (layer F.Cu) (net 6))
 (segment (start 129.869999 79.340001) (end 131.719999 81.190001) (width 0.5) (layer F.Cu) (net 6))
 (segment (start 131.719999 81.190001) (end 131.719999 92.440001) (width 0.5) (layer F.Cu) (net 6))
 (segment (start 131.719999 92.440001) (end 132.939998 93.66) (width 0.5) (layer F.Cu) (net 6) (status 20))
 (segment (start 132.939998 93.66) (end 133.32 93.66) (width 0.5) (layer F.Cu) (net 6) (status 30))
 (segment (start 118.21048 53.05948) (end 119.0625 53.9115) (width 0.5) (layer F.Cu) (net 6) (status 20))
 (segment (start 118.21048 51.67884) (end 118.21048 53.05948) (width 0.5) (layer F.Cu) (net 6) (status 10))
 (segment (start 119.0625 58.9915) (end 117.262488 60.791512) (width 0.5) (layer F.Cu) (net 15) (status 10))
 (segment (start 117.262488 60.791512) (end 117.262488 66.629431) (width 0.5) (layer F.Cu) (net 15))
 (segment (start 117.262488 66.629431) (end 117.446491 66.813434) (width 0.5) (layer F.Cu) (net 15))
 (segment (start 117.446491 66.813434) (end 117.446491 77.986491) (width 0.5) (layer F.Cu) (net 15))
 (segment (start 117.446491 77.986491) (end 118.12 78.66) (width 0.5) (layer F.Cu) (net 15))
 (segment (start 118.12 78.66) (end 118.12 79.66) (width 0.5) (layer F.Cu) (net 15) (status 20))
 (segment (start 119.0625 56.4515) (end 116.332 59.182) (width 0.5) (layer F.Cu) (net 14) (status 10))
 (segment (start 116.332 59.182) (end 116.332 80.9625) (width 0.5) (layer F.Cu) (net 14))
 (segment (start 117.0295 81.66) (end 118.12 81.66) (width 0.5) (layer F.Cu) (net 14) (status 30))
 (segment (start 116.332 80.9625) (end 117.0295 81.66) (width 0.5) (layer F.Cu) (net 14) (status 20))
 (via (at 133.3754 89.67216) (size 0.8) (drill 0.4) (layers F.Cu B.Cu) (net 13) (status 30))
 (via (at 134.43712 75.42276) (size 0.8) (drill 0.4) (layers F.Cu B.Cu) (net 13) (status 30))
 (segment (start 134.43712 88.61044) (end 133.3754 89.67216) (width 0.5) (layer B.Cu) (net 13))
 (segment (start 134.43712 75.42276) (end 134.43712 88.61044) (width 0.5) (layer B.Cu) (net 13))
 (segment (start 127.7874 77.0926) (end 126.72 78.16) (width 0.5) (layer F.Cu) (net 12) (status 20))
 (segment (start 127.7874 75.3488) (end 127.7874 77.0926) (width 0.5) (layer F.Cu) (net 12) (status 10))
 (segment (start 125.5268 77.3532) (end 124.72 78.16) (width 0.5) (layer F.Cu) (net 11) (status 20))
 (segment (start 125.5268 75.368) (end 125.5268 77.3532) (width 0.5) (layer F.Cu) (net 11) (status 10))
 (segment (start 124.426799 74.267999) (end 125.5268 75.368) (width 0.5) (layer F.Cu) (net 11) (status 20))
 (segment (start 124.426799 72.277997) (end 124.426799 74.267999) (width 0.5) (layer F.Cu) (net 11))
 (segment (start 124.067601 71.918799) (end 124.426799 72.277997) (width 0.5) (layer F.Cu) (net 11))
 (segment (start 120.163601 71.918799) (end 124.067601 71.918799) (width 0.5) (layer F.Cu) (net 11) (status 10))
 (via (at 125.7935 63.3095) (size 0.8) (drill 0.4) (layers F.Cu B.Cu) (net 1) (status 30))
 (via (at 124.714 64.7065) (size 0.8) (drill 0.4) (layers F.Cu B.Cu) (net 1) (status 30))
 (via (at 125.7935 64.77) (size 0.8) (drill 0.4) (layers F.Cu B.Cu) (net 1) (status 30))
 (via (at 126.9365 64.643) (size 0.8) (drill 0.4) (layers F.Cu B.Cu) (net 1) (status 30))
 (via (at 126.9365 63.373) (size 0.8) (drill 0.4) (layers F.Cu B.Cu) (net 1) (status 30))
 (via (at 124.6505 63.3095) (size 0.8) (drill 0.4) (layers F.Cu B.Cu) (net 1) (status 30))
 (segment (start 132.75 61.284) (end 132.9334 61.4674) (width 0.5) (layer B.Cu) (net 1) (status 30))
 (segment (start 132.75 59.25) (end 132.75 61.284) (width 0.5) (layer B.Cu) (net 1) (status 30))
 (segment (start 131.38408 63.01672) (end 131.38408 63.82064) (width 0.5) (layer B.Cu) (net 1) (status 30))
 (segment (start 132.9334 61.4674) (end 131.38408 63.01672) (width 0.5) (layer B.Cu) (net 1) (status 30))
 (segment (start 135.3185 64.192) (end 131.6925 64.192) (width 0.5) (layer F.Cu) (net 1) (status 10))
 (segment (start 131.6925 64.192) (end 131.445 63.9445) (width 0.5) (layer F.Cu) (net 1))
 (via (at 131.38408 63.82064) (size 0.8) (drill 0.4) (layers F.Cu B.Cu) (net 1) (status 30))
 (segment (start 126.238 53.975) (end 128.135 53.975) (width 0.5) (layer B.Cu) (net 1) (status 10))
 (segment (start 128.135 53.975) (end 132.75 58.59) (width 0.5) (layer B.Cu) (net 1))
 (segment (start 132.75 58.59) (end 132.75 59.25) (width 0.5) (layer B.Cu) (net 1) (status 20))
 (segment (start 132.75 57.1912) (end 132.75 59.25) (width 0.5) (layer B.Cu) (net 1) (status 20))
 (segment (start 134.52348 55.41772) (end 132.75 57.1912) (width 0.5) (layer B.Cu) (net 1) (status 10))
 (segment (start 126.9365 63.373) (end 128.71704 63.373) (width 0.5) (layer F.Cu) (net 1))
 (segment (start 128.71704 63.373) (end 132.77088 59.31916) (width 0.5) (layer F.Cu) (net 1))
 (segment (start 132.75 59.25) (end 132.75 59.25) (width 0.5) (layer B.Cu) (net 1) (status 20))
 (via (at 132.75 59.25) (size 0.8) (drill 0.4) (layers F.Cu B.Cu) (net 1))
 (segment (start 128.127639 59.420639) (end 126.238 57.531) (width 0.5) (layer B.Cu) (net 2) (status 20))
 (segment (start 130.034079 59.420639) (end 128.127639 59.420639) (width 0.5) (layer B.Cu) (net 2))
 (segment (start 131.38408 60.77064) (end 130.034079 59.420639) (width 0.5) (layer B.Cu) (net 2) (status 10))
 (segment (start 130.048 75.3488) (end 128.72 76.6768) (width 0.5) (layer F.Cu) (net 10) (status 10))
 (segment (start 128.72 76.6768) (end 128.72 78.16) (width 0.5) (layer F.Cu) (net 10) (status 20))
 (via (at 135.001 61.468) (size 0.8) (drill 0.4) (layers F.Cu B.Cu) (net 7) (status 30))
 (segment (start 132.328399 63.167399) (end 132.1435 63.352298) (width 0.5) (layer B.Cu) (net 7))
 (segment (start 134.003393 63.167399) (end 132.328399 63.167399) (width 0.5) (layer B.Cu) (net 7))
 (segment (start 135.001 62.169792) (end 134.003393 63.167399) (width 0.5) (layer B.Cu) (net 7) (status 10))
 (segment (start 135.001 61.468) (end 135.001 62.169792) (width 0.5) (layer B.Cu) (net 7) (status 30))
 (segment (start 129.48408 64.690632) (end 129.48408 63.82064) (width 0.5) (layer B.Cu) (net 7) (status 30))
 (segment (start 129.964098 65.17065) (end 129.48408 64.690632) (width 0.5) (layer B.Cu) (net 7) (status 20))
 (segment (start 131.989072 65.17065) (end 129.964098 65.17065) (width 0.5) (layer B.Cu) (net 7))
 (segment (start 132.1435 65.016222) (end 131.989072 65.17065) (width 0.5) (layer B.Cu) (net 7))
 (segment (start 132.1435 63.352298) (end 132.1435 65.016222) (width 0.5) (layer B.Cu) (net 7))
 (segment (start 120.8216 75.2348) (end 123.0376 73.0188) (width 0.5) (layer F.Cu) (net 3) (status 30))
 (segment (start 120.4187 75.2348) (end 120.8216 75.2348) (width 0.5) (layer F.Cu) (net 3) (status 30))
 (segment (start 123.0376 75.8424) (end 120.72 78.16) (width 0.5) (layer F.Cu) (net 8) (status 30))
 (segment (start 123.0376 75.4188) (end 123.0376 75.8424) (width 0.5) (layer F.Cu) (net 8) (status 30))
 (via (at 135.35152 51.97856) (size 0.8) (drill 0.4) (layers F.Cu B.Cu) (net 9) (status 30))
 (segment (start 135.35152 51.97856) (end 120.87352 51.97856) (width 0.5) (layer B.Cu) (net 9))
 (segment (start 120.87352 51.97856) (end 120.68302 51.78806) (width 0.5) (layer B.Cu) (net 9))
 (segment (start 120.68302 51.78806) (end 120.64492 51.74996) (width 0.5) (layer B.Cu) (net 9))
 (via (at 120.68302 51.78806) (size 0.8) (drill 0.4) (layers F.Cu B.Cu) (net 9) (status 30)))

